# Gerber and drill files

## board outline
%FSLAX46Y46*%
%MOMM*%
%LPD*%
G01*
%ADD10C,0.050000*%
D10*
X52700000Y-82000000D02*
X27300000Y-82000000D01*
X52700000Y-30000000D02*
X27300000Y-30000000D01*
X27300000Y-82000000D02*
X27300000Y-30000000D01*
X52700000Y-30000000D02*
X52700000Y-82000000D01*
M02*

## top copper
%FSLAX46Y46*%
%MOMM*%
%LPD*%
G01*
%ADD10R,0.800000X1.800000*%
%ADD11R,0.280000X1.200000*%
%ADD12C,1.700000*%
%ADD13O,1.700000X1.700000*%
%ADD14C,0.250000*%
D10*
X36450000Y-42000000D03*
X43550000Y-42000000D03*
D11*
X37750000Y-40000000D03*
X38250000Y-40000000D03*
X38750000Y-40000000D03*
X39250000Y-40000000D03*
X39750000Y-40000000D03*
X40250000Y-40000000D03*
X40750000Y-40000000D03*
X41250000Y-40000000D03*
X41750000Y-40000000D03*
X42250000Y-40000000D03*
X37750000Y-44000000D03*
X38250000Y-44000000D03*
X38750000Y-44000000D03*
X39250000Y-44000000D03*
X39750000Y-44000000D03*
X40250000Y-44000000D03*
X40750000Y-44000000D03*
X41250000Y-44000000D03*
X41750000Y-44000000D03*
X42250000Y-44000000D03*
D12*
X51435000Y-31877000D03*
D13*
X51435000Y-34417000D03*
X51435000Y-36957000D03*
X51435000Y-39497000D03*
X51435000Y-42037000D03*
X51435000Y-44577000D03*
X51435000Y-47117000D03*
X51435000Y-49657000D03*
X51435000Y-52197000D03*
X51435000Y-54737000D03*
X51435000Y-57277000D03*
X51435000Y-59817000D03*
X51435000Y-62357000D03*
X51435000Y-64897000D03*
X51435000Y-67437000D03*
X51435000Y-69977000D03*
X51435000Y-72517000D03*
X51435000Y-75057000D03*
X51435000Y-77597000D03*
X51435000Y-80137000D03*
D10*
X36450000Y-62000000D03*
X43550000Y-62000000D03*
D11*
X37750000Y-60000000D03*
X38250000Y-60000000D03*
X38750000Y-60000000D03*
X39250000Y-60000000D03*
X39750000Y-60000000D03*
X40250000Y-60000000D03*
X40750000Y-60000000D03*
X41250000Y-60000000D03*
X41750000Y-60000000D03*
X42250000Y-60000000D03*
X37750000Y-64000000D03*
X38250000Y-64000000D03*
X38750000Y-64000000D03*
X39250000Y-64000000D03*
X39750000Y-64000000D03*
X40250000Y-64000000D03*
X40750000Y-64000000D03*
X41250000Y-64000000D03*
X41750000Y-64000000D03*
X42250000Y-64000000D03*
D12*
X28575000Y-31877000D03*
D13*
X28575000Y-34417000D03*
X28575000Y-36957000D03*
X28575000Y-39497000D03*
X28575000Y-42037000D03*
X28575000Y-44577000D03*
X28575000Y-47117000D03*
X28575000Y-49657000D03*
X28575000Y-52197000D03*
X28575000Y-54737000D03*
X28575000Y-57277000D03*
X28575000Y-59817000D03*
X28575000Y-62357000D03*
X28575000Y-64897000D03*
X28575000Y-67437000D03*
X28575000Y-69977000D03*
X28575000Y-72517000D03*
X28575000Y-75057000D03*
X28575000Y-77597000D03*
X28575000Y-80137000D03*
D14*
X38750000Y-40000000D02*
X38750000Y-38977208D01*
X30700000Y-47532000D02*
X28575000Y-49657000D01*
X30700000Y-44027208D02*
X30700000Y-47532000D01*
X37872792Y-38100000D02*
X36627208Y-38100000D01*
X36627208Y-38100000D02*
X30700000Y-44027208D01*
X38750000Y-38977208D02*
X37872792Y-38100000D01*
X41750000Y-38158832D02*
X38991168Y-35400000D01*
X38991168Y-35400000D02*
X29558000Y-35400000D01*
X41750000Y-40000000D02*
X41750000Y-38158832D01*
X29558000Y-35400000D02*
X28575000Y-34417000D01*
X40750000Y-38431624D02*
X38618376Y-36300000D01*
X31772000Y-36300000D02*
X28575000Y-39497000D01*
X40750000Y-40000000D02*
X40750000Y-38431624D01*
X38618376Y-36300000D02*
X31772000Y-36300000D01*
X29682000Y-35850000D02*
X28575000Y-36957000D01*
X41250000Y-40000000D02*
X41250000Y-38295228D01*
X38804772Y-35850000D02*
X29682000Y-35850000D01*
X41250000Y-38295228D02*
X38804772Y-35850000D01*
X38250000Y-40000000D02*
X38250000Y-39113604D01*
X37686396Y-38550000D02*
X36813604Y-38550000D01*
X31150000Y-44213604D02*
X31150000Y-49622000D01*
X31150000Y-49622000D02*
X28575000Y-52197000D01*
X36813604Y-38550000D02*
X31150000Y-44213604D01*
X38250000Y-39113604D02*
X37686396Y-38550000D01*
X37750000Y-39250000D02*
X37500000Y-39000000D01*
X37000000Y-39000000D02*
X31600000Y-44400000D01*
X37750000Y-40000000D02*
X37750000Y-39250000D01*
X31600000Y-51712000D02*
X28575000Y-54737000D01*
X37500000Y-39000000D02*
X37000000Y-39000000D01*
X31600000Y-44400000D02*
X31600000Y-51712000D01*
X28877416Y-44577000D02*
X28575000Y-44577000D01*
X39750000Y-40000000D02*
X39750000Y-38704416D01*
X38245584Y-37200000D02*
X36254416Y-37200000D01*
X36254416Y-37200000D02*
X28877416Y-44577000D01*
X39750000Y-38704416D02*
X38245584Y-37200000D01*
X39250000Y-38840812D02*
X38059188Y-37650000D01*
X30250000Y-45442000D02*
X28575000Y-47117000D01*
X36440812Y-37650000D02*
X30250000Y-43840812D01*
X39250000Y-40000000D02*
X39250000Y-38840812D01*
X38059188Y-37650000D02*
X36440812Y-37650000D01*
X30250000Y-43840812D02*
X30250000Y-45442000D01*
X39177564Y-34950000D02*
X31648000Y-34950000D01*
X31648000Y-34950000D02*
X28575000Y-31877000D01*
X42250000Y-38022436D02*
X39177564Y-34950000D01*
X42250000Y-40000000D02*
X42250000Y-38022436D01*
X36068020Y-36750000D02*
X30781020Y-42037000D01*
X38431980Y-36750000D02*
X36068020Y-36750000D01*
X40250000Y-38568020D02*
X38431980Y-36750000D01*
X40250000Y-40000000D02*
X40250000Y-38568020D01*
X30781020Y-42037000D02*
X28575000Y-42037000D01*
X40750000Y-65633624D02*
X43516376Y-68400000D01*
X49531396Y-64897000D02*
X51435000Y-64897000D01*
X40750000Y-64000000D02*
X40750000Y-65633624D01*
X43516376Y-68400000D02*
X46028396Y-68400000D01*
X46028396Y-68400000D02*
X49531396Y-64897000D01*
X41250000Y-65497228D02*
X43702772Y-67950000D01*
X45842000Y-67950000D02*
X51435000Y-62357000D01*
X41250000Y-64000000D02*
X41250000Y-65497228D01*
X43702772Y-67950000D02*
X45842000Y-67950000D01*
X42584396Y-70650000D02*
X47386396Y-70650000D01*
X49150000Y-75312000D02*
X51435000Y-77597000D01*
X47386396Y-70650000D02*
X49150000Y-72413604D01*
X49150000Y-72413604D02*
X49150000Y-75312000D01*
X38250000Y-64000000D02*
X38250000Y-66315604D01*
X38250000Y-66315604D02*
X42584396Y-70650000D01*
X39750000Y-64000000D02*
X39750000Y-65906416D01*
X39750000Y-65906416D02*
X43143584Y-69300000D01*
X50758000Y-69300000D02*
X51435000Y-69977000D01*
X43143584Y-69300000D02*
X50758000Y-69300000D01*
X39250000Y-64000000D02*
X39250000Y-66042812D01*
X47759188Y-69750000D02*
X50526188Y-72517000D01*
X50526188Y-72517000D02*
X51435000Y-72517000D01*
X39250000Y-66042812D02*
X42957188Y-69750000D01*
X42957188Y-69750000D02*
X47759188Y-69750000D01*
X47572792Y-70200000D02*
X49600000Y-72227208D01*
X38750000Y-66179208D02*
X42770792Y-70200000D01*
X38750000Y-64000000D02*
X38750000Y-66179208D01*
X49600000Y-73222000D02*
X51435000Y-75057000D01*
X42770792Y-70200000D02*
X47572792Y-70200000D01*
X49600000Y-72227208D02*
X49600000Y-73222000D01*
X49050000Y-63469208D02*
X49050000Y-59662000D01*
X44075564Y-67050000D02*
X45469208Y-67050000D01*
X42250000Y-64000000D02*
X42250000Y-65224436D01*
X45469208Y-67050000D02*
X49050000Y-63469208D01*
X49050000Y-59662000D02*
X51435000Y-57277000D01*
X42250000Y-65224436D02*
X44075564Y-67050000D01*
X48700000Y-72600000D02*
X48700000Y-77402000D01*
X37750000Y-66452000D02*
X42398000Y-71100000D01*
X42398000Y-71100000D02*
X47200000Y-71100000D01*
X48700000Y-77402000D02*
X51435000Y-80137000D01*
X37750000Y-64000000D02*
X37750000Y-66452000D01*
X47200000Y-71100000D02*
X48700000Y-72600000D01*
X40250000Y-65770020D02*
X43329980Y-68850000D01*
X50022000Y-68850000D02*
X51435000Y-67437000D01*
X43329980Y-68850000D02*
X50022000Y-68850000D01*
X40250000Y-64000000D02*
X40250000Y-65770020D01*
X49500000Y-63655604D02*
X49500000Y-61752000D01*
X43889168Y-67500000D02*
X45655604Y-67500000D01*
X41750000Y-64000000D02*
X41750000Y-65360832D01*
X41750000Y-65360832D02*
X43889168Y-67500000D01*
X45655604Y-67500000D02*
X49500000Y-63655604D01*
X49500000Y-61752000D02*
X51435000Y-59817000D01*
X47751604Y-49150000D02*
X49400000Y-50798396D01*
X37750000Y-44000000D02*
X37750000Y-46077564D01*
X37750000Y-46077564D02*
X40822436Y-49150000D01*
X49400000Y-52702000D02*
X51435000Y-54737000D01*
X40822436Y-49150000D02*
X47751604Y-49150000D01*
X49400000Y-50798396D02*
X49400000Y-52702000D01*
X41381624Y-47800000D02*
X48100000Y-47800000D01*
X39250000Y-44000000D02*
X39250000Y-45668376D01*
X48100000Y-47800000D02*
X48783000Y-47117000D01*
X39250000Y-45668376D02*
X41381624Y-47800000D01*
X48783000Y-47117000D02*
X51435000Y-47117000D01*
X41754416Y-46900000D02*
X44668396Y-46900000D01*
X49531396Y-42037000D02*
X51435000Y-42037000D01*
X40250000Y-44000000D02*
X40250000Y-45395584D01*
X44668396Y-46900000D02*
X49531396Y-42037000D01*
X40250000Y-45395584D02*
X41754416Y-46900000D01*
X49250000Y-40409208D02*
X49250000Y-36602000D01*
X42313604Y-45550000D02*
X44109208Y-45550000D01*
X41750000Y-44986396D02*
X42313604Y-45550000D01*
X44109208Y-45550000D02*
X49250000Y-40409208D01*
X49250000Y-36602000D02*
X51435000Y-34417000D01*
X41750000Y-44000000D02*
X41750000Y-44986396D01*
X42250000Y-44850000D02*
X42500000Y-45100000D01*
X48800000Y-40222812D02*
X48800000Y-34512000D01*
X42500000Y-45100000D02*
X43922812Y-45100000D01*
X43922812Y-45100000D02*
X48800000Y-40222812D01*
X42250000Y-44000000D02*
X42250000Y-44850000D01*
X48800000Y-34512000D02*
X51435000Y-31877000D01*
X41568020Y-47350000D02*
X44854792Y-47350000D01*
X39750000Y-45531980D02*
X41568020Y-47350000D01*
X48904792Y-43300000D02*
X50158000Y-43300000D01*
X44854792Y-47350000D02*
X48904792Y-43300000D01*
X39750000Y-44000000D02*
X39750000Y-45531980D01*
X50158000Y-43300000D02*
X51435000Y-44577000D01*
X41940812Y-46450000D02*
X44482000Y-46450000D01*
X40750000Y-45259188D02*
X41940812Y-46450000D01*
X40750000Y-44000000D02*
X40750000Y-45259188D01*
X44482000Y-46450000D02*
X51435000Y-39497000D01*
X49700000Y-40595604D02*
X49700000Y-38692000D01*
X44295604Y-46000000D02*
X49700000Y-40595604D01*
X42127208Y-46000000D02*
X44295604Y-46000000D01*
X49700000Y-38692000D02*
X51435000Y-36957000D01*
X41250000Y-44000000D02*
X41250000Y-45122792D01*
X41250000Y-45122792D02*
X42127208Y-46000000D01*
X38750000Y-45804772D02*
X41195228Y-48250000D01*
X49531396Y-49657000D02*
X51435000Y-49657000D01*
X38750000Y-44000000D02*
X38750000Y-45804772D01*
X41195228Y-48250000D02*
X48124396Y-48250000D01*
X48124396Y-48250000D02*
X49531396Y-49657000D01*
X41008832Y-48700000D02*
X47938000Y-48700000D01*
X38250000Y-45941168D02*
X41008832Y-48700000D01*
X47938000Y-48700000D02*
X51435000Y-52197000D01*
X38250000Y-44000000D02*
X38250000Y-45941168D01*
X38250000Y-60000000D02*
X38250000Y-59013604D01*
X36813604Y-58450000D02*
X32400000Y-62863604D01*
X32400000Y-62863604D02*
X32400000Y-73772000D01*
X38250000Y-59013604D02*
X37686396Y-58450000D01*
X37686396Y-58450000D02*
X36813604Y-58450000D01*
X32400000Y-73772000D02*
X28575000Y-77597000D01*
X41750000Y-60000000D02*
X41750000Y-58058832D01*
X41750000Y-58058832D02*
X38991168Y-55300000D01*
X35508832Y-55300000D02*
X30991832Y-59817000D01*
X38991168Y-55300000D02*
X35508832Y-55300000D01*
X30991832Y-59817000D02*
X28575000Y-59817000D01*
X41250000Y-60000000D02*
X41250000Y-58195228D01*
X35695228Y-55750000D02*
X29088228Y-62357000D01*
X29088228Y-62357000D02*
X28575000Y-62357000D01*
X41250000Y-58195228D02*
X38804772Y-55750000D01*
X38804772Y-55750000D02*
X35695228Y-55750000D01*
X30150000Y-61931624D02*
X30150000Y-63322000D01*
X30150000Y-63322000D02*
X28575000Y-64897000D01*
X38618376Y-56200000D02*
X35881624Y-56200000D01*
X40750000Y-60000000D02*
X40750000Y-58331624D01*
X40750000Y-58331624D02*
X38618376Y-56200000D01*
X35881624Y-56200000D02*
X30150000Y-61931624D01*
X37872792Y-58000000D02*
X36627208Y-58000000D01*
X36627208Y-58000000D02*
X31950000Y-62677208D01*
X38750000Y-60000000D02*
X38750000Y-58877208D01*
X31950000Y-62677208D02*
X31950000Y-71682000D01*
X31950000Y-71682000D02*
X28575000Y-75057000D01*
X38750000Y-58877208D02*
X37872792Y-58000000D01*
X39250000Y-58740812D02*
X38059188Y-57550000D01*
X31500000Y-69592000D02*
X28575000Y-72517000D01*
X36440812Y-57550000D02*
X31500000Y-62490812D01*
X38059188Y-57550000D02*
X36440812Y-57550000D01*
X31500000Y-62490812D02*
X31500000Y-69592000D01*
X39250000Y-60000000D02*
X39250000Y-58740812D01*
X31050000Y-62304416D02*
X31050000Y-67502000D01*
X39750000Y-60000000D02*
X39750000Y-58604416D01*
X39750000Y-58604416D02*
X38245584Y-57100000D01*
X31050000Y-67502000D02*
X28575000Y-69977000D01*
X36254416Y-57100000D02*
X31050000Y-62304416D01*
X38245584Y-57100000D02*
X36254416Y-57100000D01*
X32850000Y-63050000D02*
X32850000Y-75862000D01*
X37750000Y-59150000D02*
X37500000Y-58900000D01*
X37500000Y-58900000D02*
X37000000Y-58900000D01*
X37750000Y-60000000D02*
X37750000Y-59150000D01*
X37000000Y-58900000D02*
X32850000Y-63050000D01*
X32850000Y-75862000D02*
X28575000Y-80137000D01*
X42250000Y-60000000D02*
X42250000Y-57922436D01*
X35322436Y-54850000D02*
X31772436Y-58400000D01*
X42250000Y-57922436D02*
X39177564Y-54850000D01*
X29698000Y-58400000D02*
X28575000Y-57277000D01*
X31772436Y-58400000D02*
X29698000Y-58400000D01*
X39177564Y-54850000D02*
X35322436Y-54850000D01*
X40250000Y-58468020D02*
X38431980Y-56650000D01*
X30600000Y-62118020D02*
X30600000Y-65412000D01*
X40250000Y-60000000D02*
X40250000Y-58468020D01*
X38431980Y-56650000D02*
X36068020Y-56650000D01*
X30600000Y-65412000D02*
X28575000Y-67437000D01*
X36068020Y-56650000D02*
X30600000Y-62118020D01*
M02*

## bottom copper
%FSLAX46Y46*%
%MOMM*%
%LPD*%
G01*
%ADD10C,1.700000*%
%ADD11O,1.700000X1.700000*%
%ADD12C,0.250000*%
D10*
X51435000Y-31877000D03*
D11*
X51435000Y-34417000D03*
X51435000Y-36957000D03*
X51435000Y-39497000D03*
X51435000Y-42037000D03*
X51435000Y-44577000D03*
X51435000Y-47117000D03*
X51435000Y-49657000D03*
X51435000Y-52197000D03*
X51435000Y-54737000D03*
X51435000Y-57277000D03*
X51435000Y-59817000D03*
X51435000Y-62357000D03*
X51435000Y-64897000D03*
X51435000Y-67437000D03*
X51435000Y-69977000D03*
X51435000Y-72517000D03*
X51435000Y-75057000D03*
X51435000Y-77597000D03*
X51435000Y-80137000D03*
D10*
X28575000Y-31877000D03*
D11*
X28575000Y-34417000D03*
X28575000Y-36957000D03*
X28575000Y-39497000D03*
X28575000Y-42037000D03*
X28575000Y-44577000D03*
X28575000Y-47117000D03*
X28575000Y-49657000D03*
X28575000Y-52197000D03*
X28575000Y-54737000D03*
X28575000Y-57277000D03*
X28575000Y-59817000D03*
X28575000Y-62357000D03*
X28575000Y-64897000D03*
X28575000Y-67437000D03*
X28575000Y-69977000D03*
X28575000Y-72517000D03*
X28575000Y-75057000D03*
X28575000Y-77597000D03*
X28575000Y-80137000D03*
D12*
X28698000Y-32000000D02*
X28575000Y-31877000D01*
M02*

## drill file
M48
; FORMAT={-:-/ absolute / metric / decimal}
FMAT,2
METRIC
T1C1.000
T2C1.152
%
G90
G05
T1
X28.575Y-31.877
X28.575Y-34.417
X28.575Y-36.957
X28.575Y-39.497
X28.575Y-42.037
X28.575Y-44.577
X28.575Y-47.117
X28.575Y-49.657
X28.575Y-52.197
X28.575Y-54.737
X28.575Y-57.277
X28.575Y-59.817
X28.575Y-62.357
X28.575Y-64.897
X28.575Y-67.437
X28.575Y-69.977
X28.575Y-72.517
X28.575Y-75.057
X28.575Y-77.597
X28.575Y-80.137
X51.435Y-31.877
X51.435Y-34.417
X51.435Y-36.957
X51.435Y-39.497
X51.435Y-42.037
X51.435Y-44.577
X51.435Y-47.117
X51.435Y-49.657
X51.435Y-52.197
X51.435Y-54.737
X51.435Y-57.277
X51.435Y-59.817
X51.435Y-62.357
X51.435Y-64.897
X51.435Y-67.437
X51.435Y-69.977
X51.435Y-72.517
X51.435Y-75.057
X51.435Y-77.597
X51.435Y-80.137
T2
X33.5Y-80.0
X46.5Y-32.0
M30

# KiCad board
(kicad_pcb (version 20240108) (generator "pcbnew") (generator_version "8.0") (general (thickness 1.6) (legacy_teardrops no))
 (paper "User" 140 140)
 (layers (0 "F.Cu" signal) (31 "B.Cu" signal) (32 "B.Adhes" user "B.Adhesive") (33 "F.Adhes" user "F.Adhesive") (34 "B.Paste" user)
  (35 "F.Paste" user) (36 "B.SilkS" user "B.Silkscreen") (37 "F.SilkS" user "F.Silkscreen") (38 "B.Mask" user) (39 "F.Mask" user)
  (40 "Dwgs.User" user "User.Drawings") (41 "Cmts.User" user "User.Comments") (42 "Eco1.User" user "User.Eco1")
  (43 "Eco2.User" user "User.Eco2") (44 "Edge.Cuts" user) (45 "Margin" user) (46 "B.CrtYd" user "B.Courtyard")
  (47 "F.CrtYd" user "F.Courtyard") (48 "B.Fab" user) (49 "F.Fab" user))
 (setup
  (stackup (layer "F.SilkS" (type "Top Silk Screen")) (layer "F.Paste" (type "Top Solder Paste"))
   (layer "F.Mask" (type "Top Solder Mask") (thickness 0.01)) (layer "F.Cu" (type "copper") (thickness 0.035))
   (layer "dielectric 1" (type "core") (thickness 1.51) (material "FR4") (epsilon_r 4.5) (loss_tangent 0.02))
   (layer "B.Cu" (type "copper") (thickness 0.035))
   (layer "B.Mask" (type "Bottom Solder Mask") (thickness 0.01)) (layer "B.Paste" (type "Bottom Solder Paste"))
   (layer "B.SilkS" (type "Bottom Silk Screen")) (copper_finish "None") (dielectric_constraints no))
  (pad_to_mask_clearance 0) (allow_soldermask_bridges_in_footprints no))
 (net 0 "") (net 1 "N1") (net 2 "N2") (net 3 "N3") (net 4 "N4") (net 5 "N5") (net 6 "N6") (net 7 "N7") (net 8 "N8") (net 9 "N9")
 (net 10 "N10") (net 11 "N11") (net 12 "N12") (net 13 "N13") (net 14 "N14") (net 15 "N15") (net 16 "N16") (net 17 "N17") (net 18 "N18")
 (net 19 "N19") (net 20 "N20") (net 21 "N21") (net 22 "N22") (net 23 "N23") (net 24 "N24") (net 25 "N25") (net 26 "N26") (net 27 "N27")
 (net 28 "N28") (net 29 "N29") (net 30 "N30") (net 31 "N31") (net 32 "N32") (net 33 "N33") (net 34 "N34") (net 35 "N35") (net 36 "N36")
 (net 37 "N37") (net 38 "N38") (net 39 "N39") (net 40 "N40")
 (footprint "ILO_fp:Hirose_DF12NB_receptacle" (layer "F.Cu") (at 40 42)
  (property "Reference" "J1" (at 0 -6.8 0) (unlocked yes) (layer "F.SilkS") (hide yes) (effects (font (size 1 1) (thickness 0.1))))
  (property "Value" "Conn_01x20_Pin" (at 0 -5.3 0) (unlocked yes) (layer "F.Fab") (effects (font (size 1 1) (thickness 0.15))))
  (pad "" smd rect (at -3.55 0) (size 0.8 1.8) (layers "F.Cu" "F.Paste" "F.Mask") (thermal_bridge_angle 45))
  (pad "" smd rect (at 3.55 0) (size 0.8 1.8) (layers "F.Cu" "F.Paste" "F.Mask") (thermal_bridge_angle 45))
  (pad "1" smd rect (at -2.25 -2) (size 0.28 1.2) (layers "F.Cu" "F.Paste" "F.Mask") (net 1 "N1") (thermal_bridge_angle 45))
  (pad "2" smd rect (at -1.75 -2) (size 0.28 1.2) (layers "F.Cu" "F.Paste" "F.Mask") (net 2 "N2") (thermal_bridge_angle 45))
  (pad "3" smd rect (at -1.25 -2) (size 0.28 1.2) (layers "F.Cu" "F.Paste" "F.Mask") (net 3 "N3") (thermal_bridge_angle 45))
  (pad "4" smd rect (at -0.75 -2) (size 0.28 1.2) (layers "F.Cu" "F.Paste" "F.Mask") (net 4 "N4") (thermal_bridge_angle 45))
  (pad "5" smd rect (at -0.25 -2) (size 0.28 1.2) (layers "F.Cu" "F.Paste" "F.Mask") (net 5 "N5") (thermal_bridge_angle 45))
  (pad "6" smd rect (at 0.25 -2) (size 0.28 1.2) (layers "F.Cu" "F.Paste" "F.Mask") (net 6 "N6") (thermal_bridge_angle 45))
  (pad "7" smd rect (at 0.75 -2) (size 0.28 1.2) (layers "F.Cu" "F.Paste" "F.Mask") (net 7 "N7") (thermal_bridge_angle 45))
  (pad "8" smd rect (at 1.25 -2) (size 0.28 1.2) (layers "F.Cu" "F.Paste" "F.Mask") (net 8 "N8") (thermal_bridge_angle 45))
  (pad "9" smd rect (at 1.75 -2) (size 0.28 1.2) (layers "F.Cu" "F.Paste" "F.Mask") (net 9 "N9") (thermal_bridge_angle 45))
  (pad "10" smd rect (at 2.25 -2) (size 0.28 1.2) (layers "F.Cu" "F.Paste" "F.Mask") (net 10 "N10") (thermal_bridge_angle 45))
  (pad "11" smd rect (at -2.25 2) (size 0.28 1.2) (layers "F.Cu" "F.Paste" "F.Mask") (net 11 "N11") (thermal_bridge_angle 45))
  (pad "12" smd rect (at -1.75 2) (size 0.28 1.2) (layers "F.Cu" "F.Paste" "F.Mask") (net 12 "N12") (thermal_bridge_angle 45))
  (pad "13" smd rect (at -1.25 2) (size 0.28 1.2) (layers "F.Cu" "F.Paste" "F.Mask") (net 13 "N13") (thermal_bridge_angle 45))
  (pad "14" smd rect (at -0.75 2) (size 0.28 1.2) (layers "F.Cu" "F.Paste" "F.Mask") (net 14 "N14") (thermal_bridge_angle 45))
  (pad "15" smd rect (at -0.25 2) (size 0.28 1.2) (layers "F.Cu" "F.Paste" "F.Mask") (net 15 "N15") (thermal_bridge_angle 45))
  (pad "16" smd rect (at 0.25 2) (size 0.28 1.2) (layers "F.Cu" "F.Paste" "F.Mask") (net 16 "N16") (thermal_bridge_angle 45))
  (pad "17" smd rect (at 0.75 2) (size 0.28 1.2) (layers "F.Cu" "F.Paste" "F.Mask") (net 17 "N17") (thermal_bridge_angle 45))
  (pad "18" smd rect (at 1.25 2) (size 0.28 1.2) (layers "F.Cu" "F.Paste" "F.Mask") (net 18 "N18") (thermal_bridge_angle 45))
  (pad "19" smd rect (at 1.75 2) (size 0.28 1.2) (layers "F.Cu" "F.Paste" "F.Mask") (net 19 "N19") (thermal_bridge_angle 45))
  (pad "20" smd rect (at 2.25 2) (size 0.28 1.2) (layers "F.Cu" "F.Paste" "F.Mask") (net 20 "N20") (thermal_bridge_angle 45)))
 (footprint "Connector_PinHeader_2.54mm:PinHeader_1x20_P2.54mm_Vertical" (layer "F.Cu") (at 51.435 31.877)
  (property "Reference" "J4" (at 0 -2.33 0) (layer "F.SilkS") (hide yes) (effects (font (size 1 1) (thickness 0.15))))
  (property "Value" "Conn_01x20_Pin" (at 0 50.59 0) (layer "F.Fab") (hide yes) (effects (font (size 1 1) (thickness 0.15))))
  (pad "1" thru_hole circle (at 0 0) (size 1.7 1.7) (drill 1) (layers "*.Cu" "*.Mask") (remove_unused_layers no) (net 20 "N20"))
  (pad "2" thru_hole oval (at 0 2.54) (size 1.7 1.7) (drill 1) (layers "*.Cu" "*.Mask") (remove_unused_layers no) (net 19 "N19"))
  (pad "3" thru_hole oval (at 0 5.08) (size 1.7 1.7) (drill 1) (layers "*.Cu" "*.Mask") (remove_unused_layers no) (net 18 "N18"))
  (pad "4" thru_hole oval (at 0 7.62) (size 1.7 1.7) (drill 1) (layers "*.Cu" "*.Mask") (remove_unused_layers no) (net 17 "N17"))
  (pad "5" thru_hole oval (at 0 10.16) (size 1.7 1.7) (drill 1) (layers "*.Cu" "*.Mask") (remove_unused_layers no) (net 16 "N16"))
  (pad "6" thru_hole oval (at 0 12.7) (size 1.7 1.7) (drill 1) (layers "*.Cu" "*.Mask") (remove_unused_layers no) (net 15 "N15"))
  (pad "7" thru_hole oval (at 0 15.24) (size 1.7 1.7) (drill 1) (layers "*.Cu" "*.Mask") (remove_unused_layers no) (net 14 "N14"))
  (pad "8" thru_hole oval (at 0 17.78) (size 1.7 1.7) (drill 1) (layers "*.Cu" "*.Mask") (remove_unused_layers no) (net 13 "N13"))
  (pad "9" thru_hole oval (at 0 20.32) (size 1.7 1.7) (drill 1) (layers "*.Cu" "*.Mask") (remove_unused_layers no) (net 12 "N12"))
  (pad "10" thru_hole oval (at 0 22.86) (size 1.7 1.7) (drill 1) (layers "*.Cu" "*.Mask") (remove_unused_layers no) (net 11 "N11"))
  (pad "11" thru_hole oval (at 0 25.4) (size 1.7 1.7) (drill 1) (layers "*.Cu" "*.Mask") (remove_unused_layers no) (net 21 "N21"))
  (pad "12" thru_hole oval (at 0 27.94) (size 1.7 1.7) (drill 1) (layers "*.Cu" "*.Mask") (remove_unused_layers no) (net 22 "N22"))
  (pad "13" thru_hole oval (at 0 30.48) (size 1.7 1.7) (drill 1) (layers "*.Cu" "*.Mask") (remove_unused_layers no) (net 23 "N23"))
  (pad "14" thru_hole oval (at 0 33.02) (size 1.7 1.7) (drill 1) (layers "*.Cu" "*.Mask") (remove_unused_layers no) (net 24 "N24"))
  (pad "15" thru_hole oval (at 0 35.56) (size 1.7 1.7) (drill 1) (layers "*.Cu" "*.Mask") (remove_unused_layers no) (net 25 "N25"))
  (pad "16" thru_hole oval (at 0 38.1) (size 1.7 1.7) (drill 1) (layers "*.Cu" "*.Mask") (remove_unused_layers no) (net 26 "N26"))
  (pad "17" thru_hole oval (at 0 40.64) (size 1.7 1.7) (drill 1) (layers "*.Cu" "*.Mask") (remove_unused_layers no) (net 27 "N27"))
  (pad "18" thru_hole oval (at 0 43.18) (size 1.7 1.7) (drill 1) (layers "*.Cu" "*.Mask") (remove_unused_layers no) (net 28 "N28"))
  (pad "19" thru_hole oval (at 0 45.72) (size 1.7 1.7) (drill 1) (layers "*.Cu" "*.Mask") (remove_unused_layers no) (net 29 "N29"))
  (pad "20" thru_hole oval (at 0 48.26) (size 1.7 1.7) (drill 1) (layers "*.Cu" "*.Mask") (remove_unused_layers no) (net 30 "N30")))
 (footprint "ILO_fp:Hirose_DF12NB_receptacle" (layer "F.Cu") (at 40 62)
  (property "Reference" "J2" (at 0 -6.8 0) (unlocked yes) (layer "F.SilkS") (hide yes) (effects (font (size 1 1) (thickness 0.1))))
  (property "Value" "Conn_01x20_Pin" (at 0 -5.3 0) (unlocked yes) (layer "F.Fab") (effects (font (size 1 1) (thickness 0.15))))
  (pad "" smd rect (at -3.55 0) (size 0.8 1.8) (layers "F.Cu" "F.Paste" "F.Mask") (thermal_bridge_angle 45))
  (pad "" smd rect (at 3.55 0) (size 0.8 1.8) (layers "F.Cu" "F.Paste" "F.Mask") (thermal_bridge_angle 45))
  (pad "1" smd rect (at -2.25 -2) (size 0.28 1.2) (layers "F.Cu" "F.Paste" "F.Mask") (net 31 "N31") (thermal_bridge_angle 45))
  (pad "2" smd rect (at -1.75 -2) (size 0.28 1.2) (layers "F.Cu" "F.Paste" "F.Mask") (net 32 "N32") (thermal_bridge_angle 45))
  (pad "3" smd rect (at -1.25 -2) (size 0.28 1.2) (layers "F.Cu" "F.Paste" "F.Mask") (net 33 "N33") (thermal_bridge_angle 45))
  (pad "4" smd rect (at -0.75 -2) (size 0.28 1.2) (layers "F.Cu" "F.Paste" "F.Mask") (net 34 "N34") (thermal_bridge_angle 45))
  (pad "5" smd rect (at -0.25 -2) (size 0.28 1.2) (layers "F.Cu" "F.Paste" "F.Mask") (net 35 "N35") (thermal_bridge_angle 45))
  (pad "6" smd rect (at 0.25 -2) (size 0.28 1.2) (layers "F.Cu" "F.Paste" "F.Mask") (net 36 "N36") (thermal_bridge_angle 45))
  (pad "7" smd rect (at 0.75 -2) (size 0.28 1.2) (layers "F.Cu" "F.Paste" "F.Mask") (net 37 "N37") (thermal_bridge_angle 45))
  (pad "8" smd rect (at 1.25 -2) (size 0.28 1.2) (layers "F.Cu" "F.Paste" "F.Mask") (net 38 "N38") (thermal_bridge_angle 45))
  (pad "9" smd rect (at 1.75 -2) (size 0.28 1.2) (layers "F.Cu" "F.Paste" "F.Mask") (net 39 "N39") (thermal_bridge_angle 45))
  (pad "10" smd rect (at 2.25 -2) (size 0.28 1.2) (layers "F.Cu" "F.Paste" "F.Mask") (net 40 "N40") (thermal_bridge_angle 45))
  (pad "11" smd rect (at -2.25 2) (size 0.28 1.2) (layers "F.Cu" "F.Paste" "F.Mask") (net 30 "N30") (thermal_bridge_angle 45))
  (pad "12" smd rect (at -1.75 2) (size 0.28 1.2) (layers "F.Cu" "F.Paste" "F.Mask") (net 29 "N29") (thermal_bridge_angle 45))
  (pad "13" smd rect (at -1.25 2) (size 0.28 1.2) (layers "F.Cu" "F.Paste" "F.Mask") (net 28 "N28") (thermal_bridge_angle 45))
  (pad "14" smd rect (at -0.75 2) (size 0.28 1.2) (layers "F.Cu" "F.Paste" "F.Mask") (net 27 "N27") (thermal_bridge_angle 45))
  (pad "15" smd rect (at -0.25 2) (size 0.28 1.2) (layers "F.Cu" "F.Paste" "F.Mask") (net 26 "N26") (thermal_bridge_angle 45))
  (pad "16" smd rect (at 0.25 2) (size 0.28 1.2) (layers "F.Cu" "F.Paste" "F.Mask") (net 25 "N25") (thermal_bridge_angle 45))
  (pad "17" smd rect (at 0.75 2) (size 0.28 1.2) (layers "F.Cu" "F.Paste" "F.Mask") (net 24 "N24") (thermal_bridge_angle 45))
  (pad "18" smd rect (at 1.25 2) (size 0.28 1.2) (layers "F.Cu" "F.Paste" "F.Mask") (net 23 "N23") (thermal_bridge_angle 45))
  (pad "19" smd rect (at 1.75 2) (size 0.28 1.2) (layers "F.Cu" "F.Paste" "F.Mask") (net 22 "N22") (thermal_bridge_angle 45))
  (pad "20" smd rect (at 2.25 2) (size 0.28 1.2) (layers "F.Cu" "F.Paste" "F.Mask") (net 21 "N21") (thermal_bridge_angle 45)))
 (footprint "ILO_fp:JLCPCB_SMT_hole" (layer "F.Cu") (at 33.5 80)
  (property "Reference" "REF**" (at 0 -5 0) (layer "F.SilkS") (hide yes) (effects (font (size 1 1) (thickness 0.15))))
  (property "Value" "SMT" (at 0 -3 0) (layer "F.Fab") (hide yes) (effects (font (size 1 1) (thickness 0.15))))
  (pad "" np_thru_hole circle (at 0 0) (size 1.152 1.152) (drill 1.152) (layers "F&B.Cu" "*.Mask") (solder_mask_margin 0.148)))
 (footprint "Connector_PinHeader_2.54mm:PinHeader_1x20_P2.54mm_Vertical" (layer "F.Cu") (at 28.575 31.877)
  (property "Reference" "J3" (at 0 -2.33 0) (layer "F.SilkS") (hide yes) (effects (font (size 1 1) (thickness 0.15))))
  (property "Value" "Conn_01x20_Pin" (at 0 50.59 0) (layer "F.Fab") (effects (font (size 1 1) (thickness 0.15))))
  (pad "1" thru_hole circle (at 0 0) (size 1.7 1.7) (drill 1) (layers "*.Cu" "*.Mask") (remove_unused_layers no) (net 10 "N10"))
  (pad "2" thru_hole oval (at 0 2.54) (size 1.7 1.7) (drill 1) (layers "*.Cu" "*.Mask") (remove_unused_layers no) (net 9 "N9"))
  (pad "3" thru_hole oval (at 0 5.08) (size 1.7 1.7) (drill 1) (layers "*.Cu" "*.Mask") (remove_unused_layers no) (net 8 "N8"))
  (pad "4" thru_hole oval (at 0 7.62) (size 1.7 1.7) (drill 1) (layers "*.Cu" "*.Mask") (remove_unused_layers no) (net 7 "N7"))
  (pad "5" thru_hole oval (at 0 10.16) (size 1.7 1.7) (drill 1) (layers "*.Cu" "*.Mask") (remove_unused_layers no) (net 6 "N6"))
  (pad "6" thru_hole oval (at 0 12.7) (size 1.7 1.7) (drill 1) (layers "*.Cu" "*.Mask") (remove_unused_layers no) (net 5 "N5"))
  (pad "7" thru_hole oval (at 0 15.24) (size 1.7 1.7) (drill 1) (layers "*.Cu" "*.Mask") (remove_unused_layers no) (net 4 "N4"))
  (pad "8" thru_hole oval (at 0 17.78) (size 1.7 1.7) (drill 1) (layers "*.Cu" "*.Mask") (remove_unused_layers no) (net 3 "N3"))
  (pad "9" thru_hole oval (at 0 20.32) (size 1.7 1.7) (drill 1) (layers "*.Cu" "*.Mask") (remove_unused_layers no) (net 2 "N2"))
  (pad "10" thru_hole oval (at 0 22.86) (size 1.7 1.7) (drill 1) (layers "*.Cu" "*.Mask") (remove_unused_layers no) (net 1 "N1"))
  (pad "11" thru_hole oval (at 0 25.4) (size 1.7 1.7) (drill 1) (layers "*.Cu" "*.Mask") (remove_unused_layers no) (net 40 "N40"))
  (pad "12" thru_hole oval (at 0 27.94) (size 1.7 1.7) (drill 1) (layers "*.Cu" "*.Mask") (remove_unused_layers no) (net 39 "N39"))
  (pad "13" thru_hole oval (at 0 30.48) (size 1.7 1.7) (drill 1) (layers "*.Cu" "*.Mask") (remove_unused_layers no) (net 38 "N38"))
  (pad "14" thru_hole oval (at 0 33.02) (size 1.7 1.7) (drill 1) (layers "*.Cu" "*.Mask") (remove_unused_layers no) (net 37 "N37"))
  (pad "15" thru_hole oval (at 0 35.56) (size 1.7 1.7) (drill 1) (layers "*.Cu" "*.Mask") (remove_unused_layers no) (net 36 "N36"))
  (pad "16" thru_hole oval (at 0 38.1) (size 1.7 1.7) (drill 1) (layers "*.Cu" "*.Mask") (remove_unused_layers no) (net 35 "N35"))
  (pad "17" thru_hole oval (at 0 40.64) (size 1.7 1.7) (drill 1) (layers "*.Cu" "*.Mask") (remove_unused_layers no) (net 34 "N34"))
  (pad "18" thru_hole oval (at 0 43.18) (size 1.7 1.7) (drill 1) (layers "*.Cu" "*.Mask") (remove_unused_layers no) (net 33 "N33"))
  (pad "19" thru_hole oval (at 0 45.72) (size 1.7 1.7) (drill 1) (layers "*.Cu" "*.Mask") (remove_unused_layers no) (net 32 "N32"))
  (pad "20" thru_hole oval (at 0 48.26) (size 1.7 1.7) (drill 1) (layers "*.Cu" "*.Mask") (remove_unused_layers no) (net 31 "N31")))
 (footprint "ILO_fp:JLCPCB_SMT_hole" (layer "F.Cu") (at 46.5 32)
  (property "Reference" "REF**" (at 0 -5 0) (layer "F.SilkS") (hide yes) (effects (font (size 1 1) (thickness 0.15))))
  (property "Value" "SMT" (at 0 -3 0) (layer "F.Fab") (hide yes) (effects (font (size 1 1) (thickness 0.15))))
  (pad "" np_thru_hole circle (at 0 0) (size 1.152 1.152) (drill 1.152) (layers "F&B.Cu" "*.Mask") (solder_mask_margin 0.148)))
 (gr_line (start 52.7 82) (end 27.3 82) (stroke (width 0.05) (type default)) (layer "Edge.Cuts"))
 (gr_line (start 52.7 30) (end 27.3 30) (stroke (width 0.05) (type default)) (layer "Edge.Cuts"))
 (gr_line (start 27.3 82) (end 27.3 30) (stroke (width 0.05) (type default)) (layer "Edge.Cuts"))
 (gr_line (start 52.7 30) (end 52.7 82) (stroke (width 0.05) (type default)) (layer "Edge.Cuts"))
 (segment (start 38.75 40) (end 38.75 38.977208) (width 0.25) (layer "F.Cu") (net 3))
 (segment (start 30.7 47.532) (end 28.575 49.657) (width 0.25) (layer "F.Cu") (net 3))
 (segment (start 30.7 44.027208) (end 30.7 47.532) (width 0.25) (layer "F.Cu") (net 3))
 (segment (start 37.872792 38.1) (end 36.627208 38.1) (width 0.25) (layer "F.Cu") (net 3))
 (segment (start 36.627208 38.1) (end 30.7 44.027208) (width 0.25) (layer "F.Cu") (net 3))
 (segment (start 38.75 38.977208) (end 37.872792 38.1) (width 0.25) (layer "F.Cu") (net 3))
 (segment (start 41.75 38.158832) (end 38.991168 35.4) (width 0.25) (layer "F.Cu") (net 9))
 (segment (start 38.991168 35.4) (end 29.558 35.4) (width 0.25) (layer "F.Cu") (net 9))
 (segment (start 41.75 40) (end 41.75 38.158832) (width 0.25) (layer "F.Cu") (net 9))
 (segment (start 29.558 35.4) (end 28.575 34.417) (width 0.25) (layer "F.Cu") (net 9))
 (segment (start 40.75 38.431624) (end 38.618376 36.3) (width 0.25) (layer "F.Cu") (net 7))
 (segment (start 31.772 36.3) (end 28.575 39.497) (width 0.25) (layer "F.Cu") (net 7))
 (segment (start 40.75 40) (end 40.75 38.431624) (width 0.25) (layer "F.Cu") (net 7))
 (segment (start 38.618376 36.3) (end 31.772 36.3) (width 0.25) (layer "F.Cu") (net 7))
 (segment (start 29.682 35.85) (end 28.575 36.957) (width 0.25) (layer "F.Cu") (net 8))
 (segment (start 41.25 40) (end 41.25 38.295228) (width 0.25) (layer "F.Cu") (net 8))
 (segment (start 38.804772 35.85) (end 29.682 35.85) (width 0.25) (layer "F.Cu") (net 8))
 (segment (start 41.25 38.295228) (end 38.804772 35.85) (width 0.25) (layer "F.Cu") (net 8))
 (segment (start 38.25 40) (end 38.25 39.113604) (width 0.25) (layer "F.Cu") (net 2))
 (segment (start 37.686396 38.55) (end 36.813604 38.55) (width 0.25) (layer "F.Cu") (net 2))
 (segment (start 31.15 44.213604) (end 31.15 49.622) (width 0.25) (layer "F.Cu") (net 2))
 (segment (start 31.15 49.622) (end 28.575 52.197) (width 0.25) (layer "F.Cu") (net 2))
 (segment (start 36.813604 38.55) (end 31.15 44.213604) (width 0.25) (layer "F.Cu") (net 2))
 (segment (start 38.25 39.113604) (end 37.686396 38.55) (width 0.25) (layer "F.Cu") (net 2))
 (segment (start 37.75 39.25) (end 37.5 39) (width 0.25) (layer "F.Cu") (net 1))
 (segment (start 37 39) (end 31.6 44.4) (width 0.25) (layer "F.Cu") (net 1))
 (segment (start 37.75 40) (end 37.75 39.25) (width 0.25) (layer "F.Cu") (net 1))
 (segment (start 31.6 51.712) (end 28.575 54.737) (width 0.25) (layer "F.Cu") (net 1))
 (segment (start 37.5 39) (end 37 39) (width 0.25) (layer "F.Cu") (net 1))
 (segment (start 31.6 44.4) (end 31.6 51.712) (width 0.25) (layer "F.Cu") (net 1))
 (segment (start 28.877416 44.577) (end 28.575 44.577) (width 0.25) (layer "F.Cu") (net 5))
 (segment (start 39.75 40) (end 39.75 38.704416) (width 0.25) (layer "F.Cu") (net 5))
 (segment (start 38.245584 37.2) (end 36.254416 37.2) (width 0.25) (layer "F.Cu") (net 5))
 (segment (start 36.254416 37.2) (end 28.877416 44.577) (width 0.25) (layer "F.Cu") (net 5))
 (segment (start 39.75 38.704416) (end 38.245584 37.2) (width 0.25) (layer "F.Cu") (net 5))
 (segment (start 39.25 38.840812) (end 38.059188 37.65) (width 0.25) (layer "F.Cu") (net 4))
 (segment (start 30.25 45.442) (end 28.575 47.117) (width 0.25) (layer "F.Cu") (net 4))
 (segment (start 36.440812 37.65) (end 30.25 43.840812) (width 0.25) (layer "F.Cu") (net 4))
 (segment (start 39.25 40) (end 39.25 38.840812) (width 0.25) (layer "F.Cu") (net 4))
 (segment (start 38.059188 37.65) (end 36.440812 37.65) (width 0.25) (layer "F.Cu") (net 4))
 (segment (start 30.25 43.840812) (end 30.25 45.442) (width 0.25) (layer "F.Cu") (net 4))
 (segment (start 39.177564 34.95) (end 31.648 34.95) (width 0.25) (layer "F.Cu") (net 10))
 (segment (start 31.648 34.95) (end 28.575 31.877) (width 0.25) (layer "F.Cu") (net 10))
 (segment (start 42.25 38.022436) (end 39.177564 34.95) (width 0.25) (layer "F.Cu") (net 10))
 (segment (start 42.25 40) (end 42.25 38.022436) (width 0.25) (layer "F.Cu") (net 10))
 (segment (start 28.698 32) (end 28.575 31.877) (width 0.25) (layer "B.Cu") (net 10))
 (segment (start 36.06802 36.75) (end 30.78102 42.037) (width 0.25) (layer "F.Cu") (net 6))
 (segment (start 38.43198 36.75) (end 36.06802 36.75) (width 0.25) (layer "F.Cu") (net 6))
 (segment (start 40.25 38.56802) (end 38.43198 36.75) (width 0.25) (layer "F.Cu") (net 6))
 (segment (start 40.25 40) (end 40.25 38.56802) (width 0.25) (layer "F.Cu") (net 6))
 (segment (start 30.78102 42.037) (end 28.575 42.037) (width 0.25) (layer "F.Cu") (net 6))
 (segment (start 40.75 65.633624) (end 43.516376 68.4) (width 0.25) (layer "F.Cu") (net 24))
 (segment (start 49.531396 64.897) (end 51.435 64.897) (width 0.25) (layer "F.Cu") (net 24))
 (segment (start 40.75 64) (end 40.75 65.633624) (width 0.25) (layer "F.Cu") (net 24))
 (segment (start 43.516376 68.4) (end 46.028396 68.4) (width 0.25) (layer "F.Cu") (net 24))
 (segment (start 46.028396 68.4) (end 49.531396 64.897) (width 0.25) (layer "F.Cu") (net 24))
 (segment (start 41.25 65.497228) (end 43.702772 67.95) (width 0.25) (layer "F.Cu") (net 23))
 (segment (start 45.842 67.95) (end 51.435 62.357) (width 0.25) (layer "F.Cu") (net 23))
 (segment (start 41.25 64) (end 41.25 65.497228) (width 0.25) (layer "F.Cu") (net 23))
 (segment (start 43.702772 67.95) (end 45.842 67.95) (width 0.25) (layer "F.Cu") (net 23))
 (segment (start 42.584396 70.65) (end 47.386396 70.65) (width 0.25) (layer "F.Cu") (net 29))
 (segment (start 49.15 75.312) (end 51.435 77.597) (width 0.25) (layer "F.Cu") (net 29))
 (segment (start 47.386396 70.65) (end 49.15 72.413604) (width 0.25) (layer "F.Cu") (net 29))
 (segment (start 49.15 72.413604) (end 49.15 75.312) (width 0.25) (layer "F.Cu") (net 29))
 (segment (start 38.25 64) (end 38.25 66.315604) (width 0.25) (layer "F.Cu") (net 29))
 (segment (start 38.25 66.315604) (end 42.584396 70.65) (width 0.25) (layer "F.Cu") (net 29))
 (segment (start 39.75 64) (end 39.75 65.906416) (width 0.25) (layer "F.Cu") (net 26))
 (segment (start 39.75 65.906416) (end 43.143584 69.3) (width 0.25) (layer "F.Cu") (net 26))
 (segment (start 50.758 69.3) (end 51.435 69.977) (width 0.25) (layer "F.Cu") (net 26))
 (segment (start 43.143584 69.3) (end 50.758 69.3) (width 0.25) (layer "F.Cu") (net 26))
 (segment (start 39.25 64) (end 39.25 66.042812) (width 0.25) (layer "F.Cu") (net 27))
 (segment (start 47.759188 69.75) (end 50.526188 72.517) (width 0.25) (layer "F.Cu") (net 27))
 (segment (start 50.526188 72.517) (end 51.435 72.517) (width 0.25) (layer "F.Cu") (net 27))
 (segment (start 39.25 66.042812) (end 42.957188 69.75) (width 0.25) (layer "F.Cu") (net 27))
 (segment (start 42.957188 69.75) (end 47.759188 69.75) (width 0.25) (layer "F.Cu") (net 27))
 (segment (start 47.572792 70.2) (end 49.6 72.227208) (width 0.25) (layer "F.Cu") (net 28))
 (segment (start 38.75 66.179208) (end 42.770792 70.2) (width 0.25) (layer "F.Cu") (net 28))
 (segment (start 38.75 64) (end 38.75 66.179208) (width 0.25) (layer "F.Cu") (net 28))
 (segment (start 49.6 73.222) (end 51.435 75.057) (width 0.25) (layer "F.Cu") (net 28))
 (segment (start 42.770792 70.2) (end 47.572792 70.2) (width 0.25) (layer "F.Cu") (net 28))
 (segment (start 49.6 72.227208) (end 49.6 73.222) (width 0.25) (layer "F.Cu") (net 28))
 (segment (start 49.05 63.469208) (end 49.05 59.662) (width 0.25) (layer "F.Cu") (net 21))
 (segment (start 44.075564 67.05) (end 45.469208 67.05) (width 0.25) (layer "F.Cu") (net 21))
 (segment (start 42.25 64) (end 42.25 65.224436) (width 0.25) (layer "F.Cu") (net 21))
 (segment (start 45.469208 67.05) (end 49.05 63.469208) (width 0.25) (layer "F.Cu") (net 21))
 (segment (start 49.05 59.662) (end 51.435 57.277) (width 0.25) (layer "F.Cu") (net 21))
 (segment (start 42.25 65.224436) (end 44.075564 67.05) (width 0.25) (layer "F.Cu") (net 21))
 (segment (start 48.7 72.6) (end 48.7 77.402) (width 0.25) (layer "F.Cu") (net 30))
 (segment (start 37.75 66.452) (end 42.398 71.1) (width 0.25) (layer "F.Cu") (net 30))
 (segment (start 42.398 71.1) (end 47.2 71.1) (width 0.25) (layer "F.Cu") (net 30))
 (segment (start 48.7 77.402) (end 51.435 80.137) (width 0.25) (layer "F.Cu") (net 30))
 (segment (start 37.75 64) (end 37.75 66.452) (width 0.25) (layer "F.Cu") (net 30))
 (segment (start 47.2 71.1) (end 48.7 72.6) (width 0.25) (layer "F.Cu") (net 30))
 (segment (start 40.25 65.77002) (end 43.32998 68.85) (width 0.25) (layer "F.Cu") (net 25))
 (segment (start 50.022 68.85) (end 51.435 67.437) (width 0.25) (layer "F.Cu") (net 25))
 (segment (start 43.32998 68.85) (end 50.022 68.85) (width 0.25) (layer "F.Cu") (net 25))
 (segment (start 40.25 64) (end 40.25 65.77002) (width 0.25) (layer "F.Cu") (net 25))
 (segment (start 49.5 63.655604) (end 49.5 61.752) (width 0.25) (layer "F.Cu") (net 22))
 (segment (start 43.889168 67.5) (end 45.655604 67.5) (width 0.25) (layer "F.Cu") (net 22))
 (segment (start 41.75 64) (end 41.75 65.360832) (width 0.25) (layer "F.Cu") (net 22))
 (segment (start 41.75 65.360832) (end 43.889168 67.5) (width 0.25) (layer "F.Cu") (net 22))
 (segment (start 45.655604 67.5) (end 49.5 63.655604) (width 0.25) (layer "F.Cu") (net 22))
 (segment (start 49.5 61.752) (end 51.435 59.817) (width 0.25) (layer "F.Cu") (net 22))
 (segment (start 47.751604 49.15) (end 49.4 50.798396) (width 0.25) (layer "F.Cu") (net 11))
 (segment (start 37.75 44) (end 37.75 46.077564) (width 0.25) (layer "F.Cu") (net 11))
 (segment (start 37.75 46.077564) (end 40.822436 49.15) (width 0.25) (layer "F.Cu") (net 11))
 (segment (start 49.4 52.702) (end 51.435 54.737) (width 0.25) (layer "F.Cu") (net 11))
 (segment (start 40.822436 49.15) (end 47.751604 49.15) (width 0.25) (layer "F.Cu") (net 11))
 (segment (start 49.4 50.798396) (end 49.4 52.702) (width 0.25) (layer "F.Cu") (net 11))
 (segment (start 41.381624 47.8) (end 48.1 47.8) (width 0.25) (layer "F.Cu") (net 14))
 (segment (start 39.25 44) (end 39.25 45.668376) (width 0.25) (layer "F.Cu") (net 14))
 (segment (start 48.1 47.8) (end 48.783 47.117) (width 0.25) (layer "F.Cu") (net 14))
 (segment (start 39.25 45.668376) (end 41.381624 47.8) (width 0.25) (layer "F.Cu") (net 14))
 (segment (start 48.783 47.117) (end 51.435 47.117) (width 0.25) (layer "F.Cu") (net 14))
 (segment (start 41.754416 46.9) (end 44.668396 46.9) (width 0.25) (layer "F.Cu") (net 16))
 (segment (start 49.531396 42.037) (end 51.435 42.037) (width 0.25) (layer "F.Cu") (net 16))
 (segment (start 40.25 44) (end 40.25 45.395584) (width 0.25) (layer "F.Cu") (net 16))
 (segment (start 44.668396 46.9) (end 49.531396 42.037) (width 0.25) (layer "F.Cu") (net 16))
 (segment (start 40.25 45.395584) (end 41.754416 46.9) (width 0.25) (layer "F.Cu") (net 16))
 (segment (start 49.25 40.409208) (end 49.25 36.602) (width 0.25) (layer "F.Cu") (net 19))
 (segment (start 42.313604 45.55) (end 44.109208 45.55) (width 0.25) (layer "F.Cu") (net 19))
 (segment (start 41.75 44.986396) (end 42.313604 45.55) (width 0.25) (layer "F.Cu") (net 19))
 (segment (start 44.109208 45.55) (end 49.25 40.409208) (width 0.25) (layer "F.Cu") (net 19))
 (segment (start 49.25 36.602) (end 51.435 34.417) (width 0.25) (layer "F.Cu") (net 19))
 (segment (start 41.75 44) (end 41.75 44.986396) (width 0.25) (layer "F.Cu") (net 19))
 (segment (start 42.25 44.85) (end 42.5 45.1) (width 0.25) (layer "F.Cu") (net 20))
 (segment (start 48.8 40.222812) (end 48.8 34.512) (width 0.25) (layer "F.Cu") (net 20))
 (segment (start 42.5 45.1) (end 43.922812 45.1) (width 0.25) (layer "F.Cu") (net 20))
 (segment (start 43.922812 45.1) (end 48.8 40.222812) (width 0.25) (layer "F.Cu") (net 20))
 (segment (start 42.25 44) (end 42.25 44.85) (width 0.25) (layer "F.Cu") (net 20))
 (segment (start 48.8 34.512) (end 51.435 31.877) (width 0.25) (layer "F.Cu") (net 20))
 (segment (start 41.56802 47.35) (end 44.854792 47.35) (width 0.25) (layer "F.Cu") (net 15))
 (segment (start 39.75 45.53198) (end 41.56802 47.35) (width 0.25) (layer "F.Cu") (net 15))
 (segment (start 48.904792 43.3) (end 50.158 43.3) (width 0.25) (layer "F.Cu") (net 15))
 (segment (start 44.854792 47.35) (end 48.904792 43.3) (width 0.25) (layer "F.Cu") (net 15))
 (segment (start 39.75 44) (end 39.75 45.53198) (width 0.25) (layer "F.Cu") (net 15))
 (segment (start 50.158 43.3) (end 51.435 44.577) (width 0.25) (layer "F.Cu") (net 15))
 (segment (start 41.940812 46.45) (end 44.482 46.45) (width 0.25) (layer "F.Cu") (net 17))
 (segment (start 40.75 45.259188) (end 41.940812 46.45) (width 0.25) (layer "F.Cu") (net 17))
 (segment (start 40.75 44) (end 40.75 45.259188) (width 0.25) (layer "F.Cu") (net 17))
 (segment (start 44.482 46.45) (end 51.435 39.497) (width 0.25) (layer "F.Cu") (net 17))
 (segment (start 49.7 40.595604) (end 49.7 38.692) (width 0.25) (layer "F.Cu") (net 18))
 (segment (start 44.295604 46) (end 49.7 40.595604) (width 0.25) (layer "F.Cu") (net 18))
 (segment (start 42.127208 46) (end 44.295604 46) (width 0.25) (layer "F.Cu") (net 18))
 (segment (start 49.7 38.692) (end 51.435 36.957) (width 0.25) (layer "F.Cu") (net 18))
 (segment (start 41.25 44) (end 41.25 45.122792) (width 0.25) (layer "F.Cu") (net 18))
 (segment (start 41.25 45.122792) (end 42.127208 46) (width 0.25) (layer "F.Cu") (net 18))
 (segment (start 38.75 45.804772) (end 41.195228 48.25) (width 0.25) (layer "F.Cu") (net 13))
 (segment (start 49.531396 49.657) (end 51.435 49.657) (width 0.25) (layer "F.Cu") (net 13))
 (segment (start 38.75 44) (end 38.75 45.804772) (width 0.25) (layer "F.Cu") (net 13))
 (segment (start 41.195228 48.25) (end 48.124396 48.25) (width 0.25) (layer "F.Cu") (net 13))
 (segment (start 48.124396 48.25) (end 49.531396 49.657) (width 0.25) (layer "F.Cu") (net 13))
 (segment (start 41.008832 48.7) (end 47.938 48.7) (width 0.25) (layer "F.Cu") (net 12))
 (segment (start 38.25 45.941168) (end 41.008832 48.7) (width 0.25) (layer "F.Cu") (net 12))
 (segment (start 47.938 48.7) (end 51.435 52.197) (width 0.25) (layer "F.Cu") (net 12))
 (segment (start 38.25 44) (end 38.25 45.941168) (width 0.25) (layer "F.Cu") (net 12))
 (segment (start 38.25 60) (end 38.25 59.013604) (width 0.25) (layer "F.Cu") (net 32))
 (segment (start 36.813604 58.45) (end 32.4 62.863604) (width 0.25) (layer "F.Cu") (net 32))
 (segment (start 32.4 62.863604) (end 32.4 73.772) (width 0.25) (layer "F.Cu") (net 32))
 (segment (start 38.25 59.013604) (end 37.686396 58.45) (width 0.25) (layer "F.Cu") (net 32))
 (segment (start 37.686396 58.45) (end 36.813604 58.45) (width 0.25) (layer "F.Cu") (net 32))
 (segment (start 32.4 73.772) (end 28.575 77.597) (width 0.25) (layer "F.Cu") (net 32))
 (segment (start 41.75 60) (end 41.75 58.058832) (width 0.25) (layer "F.Cu") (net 39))
 (segment (start 41.75 58.058832) (end 38.991168 55.3) (width 0.25) (layer "F.Cu") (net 39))
 (segment (start 35.508832 55.3) (end 30.991832 59.817) (width 0.25) (layer "F.Cu") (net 39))
 (segment (start 38.991168 55.3) (end 35.508832 55.3) (width 0.25) (layer "F.Cu") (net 39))
 (segment (start 30.991832 59.817) (end 28.575 59.817) (width 0.25) (layer "F.Cu") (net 39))
 (segment (start 41.25 60) (end 41.25 58.195228) (width 0.25) (layer "F.Cu") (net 38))
 (segment (start 35.695228 55.75) (end 29.088228 62.357) (width 0.25) (layer "F.Cu") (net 38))
 (segment (start 29.088228 62.357) (end 28.575 62.357) (width 0.25) (layer "F.Cu") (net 38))
 (segment (start 41.25 58.195228) (end 38.804772 55.75) (width 0.25) (layer "F.Cu") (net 38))
 (segment (start 38.804772 55.75) (end 35.695228 55.75) (width 0.25) (layer "F.Cu") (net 38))
 (segment (start 30.15 61.931624) (end 30.15 63.322) (width 0.25) (layer "F.Cu") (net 37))
 (segment (start 30.15 63.322) (end 28.575 64.897) (width 0.25) (layer "F.Cu") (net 37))
 (segment (start 38.618376 56.2) (end 35.881624 56.2) (width 0.25) (layer "F.Cu") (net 37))
 (segment (start 40.75 60) (end 40.75 58.331624) (width 0.25) (layer "F.Cu") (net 37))
 (segment (start 40.75 58.331624) (end 38.618376 56.2) (width 0.25) (layer "F.Cu") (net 37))
 (segment (start 35.881624 56.2) (end 30.15 61.931624) (width 0.25) (layer "F.Cu") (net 37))
 (segment (start 37.872792 58) (end 36.627208 58) (width 0.25) (layer "F.Cu") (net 33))
 (segment (start 36.627208 58) (end 31.95 62.677208) (width 0.25) (layer "F.Cu") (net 33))
 (segment (start 38.75 60) (end 38.75 58.877208) (width 0.25) (layer "F.Cu") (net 33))
 (segment (start 31.95 62.677208) (end 31.95 71.682) (width 0.25) (layer "F.Cu") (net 33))
 (segment (start 31.95 71.682) (end 28.575 75.057) (width 0.25) (layer "F.Cu") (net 33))
 (segment (start 38.75 58.877208) (end 37.872792 58) (width 0.25) (layer "F.Cu") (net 33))
 (segment (start 39.25 58.740812) (end 38.059188 57.55) (width 0.25) (layer "F.Cu") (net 34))
 (segment (start 31.5 69.592) (end 28.575 72.517) (width 0.25) (layer "F.Cu") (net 34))
 (segment (start 36.440812 57.55) (end 31.5 62.490812) (width 0.25) (layer "F.Cu") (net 34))
 (segment (start 38.059188 57.55) (end 36.440812 57.55) (width 0.25) (layer "F.Cu") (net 34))
 (segment (start 31.5 62.490812) (end 31.5 69.592) (width 0.25) (layer "F.Cu") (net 34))
 (segment (start 39.25 60) (end 39.25 58.740812) (width 0.25) (layer "F.Cu") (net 34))
 (segment (start 31.05 62.304416) (end 31.05 67.502) (width 0.25) (layer "F.Cu") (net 35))
 (segment (start 39.75 60) (end 39.75 58.604416) (width 0.25) (layer "F.Cu") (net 35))
 (segment (start 39.75 58.604416) (end 38.245584 57.1) (width 0.25) (layer "F.Cu") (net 35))
 (segment (start 31.05 67.502) (end 28.575 69.977) (width 0.25) (layer "F.Cu") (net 35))
 (segment (start 36.254416 57.1) (end 31.05 62.304416) (width 0.25) (layer "F.Cu") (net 35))
 (segment (start 38.245584 57.1) (end 36.254416 57.1) (width 0.25) (layer "F.Cu") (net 35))
 (segment (start 32.85 63.05) (end 32.85 75.862) (width 0.25) (layer "F.Cu") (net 31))
 (segment (start 37.75 59.15) (end 37.5 58.9) (width 0.25) (layer "F.Cu") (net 31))
 (segment (start 37.5 58.9) (end 37 58.9) (width 0.25) (layer "F.Cu") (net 31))
 (segment (start 37.75 60) (end 37.75 59.15) (width 0.25) (layer "F.Cu") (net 31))
 (segment (start 37 58.9) (end 32.85 63.05) (width 0.25) (layer "F.Cu") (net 31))
 (segment (start 32.85 75.862) (end 28.575 80.137) (width 0.25) (layer "F.Cu") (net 31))
 (segment (start 42.25 60) (end 42.25 57.922436) (width 0.25) (layer "F.Cu") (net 40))
 (segment (start 35.322436 54.85) (end 31.772436 58.4) (width 0.25) (layer "F.Cu") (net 40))
 (segment (start 42.25 57.922436) (end 39.177564 54.85) (width 0.25) (layer "F.Cu") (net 40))
 (segment (start 29.698 58.4) (end 28.575 57.277) (width 0.25) (layer "F.Cu") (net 40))
 (segment (start 31.772436 58.4) (end 29.698 58.4) (width 0.25) (layer "F.Cu") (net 40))
 (segment (start 39.177564 54.85) (end 35.322436 54.85) (width 0.25) (layer "F.Cu") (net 40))
 (segment (start 40.25 58.46802) (end 38.43198 56.65) (width 0.25) (layer "F.Cu") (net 36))
 (segment (start 30.6 62.11802) (end 30.6 65.412) (width 0.25) (layer "F.Cu") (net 36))
 (segment (start 40.25 60) (end 40.25 58.46802) (width 0.25) (layer "F.Cu") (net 36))
 (segment (start 38.43198 56.65) (end 36.06802 56.65) (width 0.25) (layer "F.Cu") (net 36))
 (segment (start 30.6 65.412) (end 28.575 67.437) (width 0.25) (layer "F.Cu") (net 36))
 (segment (start 36.06802 56.65) (end 30.6 62.11802) (width 0.25) (layer "F.Cu") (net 36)))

